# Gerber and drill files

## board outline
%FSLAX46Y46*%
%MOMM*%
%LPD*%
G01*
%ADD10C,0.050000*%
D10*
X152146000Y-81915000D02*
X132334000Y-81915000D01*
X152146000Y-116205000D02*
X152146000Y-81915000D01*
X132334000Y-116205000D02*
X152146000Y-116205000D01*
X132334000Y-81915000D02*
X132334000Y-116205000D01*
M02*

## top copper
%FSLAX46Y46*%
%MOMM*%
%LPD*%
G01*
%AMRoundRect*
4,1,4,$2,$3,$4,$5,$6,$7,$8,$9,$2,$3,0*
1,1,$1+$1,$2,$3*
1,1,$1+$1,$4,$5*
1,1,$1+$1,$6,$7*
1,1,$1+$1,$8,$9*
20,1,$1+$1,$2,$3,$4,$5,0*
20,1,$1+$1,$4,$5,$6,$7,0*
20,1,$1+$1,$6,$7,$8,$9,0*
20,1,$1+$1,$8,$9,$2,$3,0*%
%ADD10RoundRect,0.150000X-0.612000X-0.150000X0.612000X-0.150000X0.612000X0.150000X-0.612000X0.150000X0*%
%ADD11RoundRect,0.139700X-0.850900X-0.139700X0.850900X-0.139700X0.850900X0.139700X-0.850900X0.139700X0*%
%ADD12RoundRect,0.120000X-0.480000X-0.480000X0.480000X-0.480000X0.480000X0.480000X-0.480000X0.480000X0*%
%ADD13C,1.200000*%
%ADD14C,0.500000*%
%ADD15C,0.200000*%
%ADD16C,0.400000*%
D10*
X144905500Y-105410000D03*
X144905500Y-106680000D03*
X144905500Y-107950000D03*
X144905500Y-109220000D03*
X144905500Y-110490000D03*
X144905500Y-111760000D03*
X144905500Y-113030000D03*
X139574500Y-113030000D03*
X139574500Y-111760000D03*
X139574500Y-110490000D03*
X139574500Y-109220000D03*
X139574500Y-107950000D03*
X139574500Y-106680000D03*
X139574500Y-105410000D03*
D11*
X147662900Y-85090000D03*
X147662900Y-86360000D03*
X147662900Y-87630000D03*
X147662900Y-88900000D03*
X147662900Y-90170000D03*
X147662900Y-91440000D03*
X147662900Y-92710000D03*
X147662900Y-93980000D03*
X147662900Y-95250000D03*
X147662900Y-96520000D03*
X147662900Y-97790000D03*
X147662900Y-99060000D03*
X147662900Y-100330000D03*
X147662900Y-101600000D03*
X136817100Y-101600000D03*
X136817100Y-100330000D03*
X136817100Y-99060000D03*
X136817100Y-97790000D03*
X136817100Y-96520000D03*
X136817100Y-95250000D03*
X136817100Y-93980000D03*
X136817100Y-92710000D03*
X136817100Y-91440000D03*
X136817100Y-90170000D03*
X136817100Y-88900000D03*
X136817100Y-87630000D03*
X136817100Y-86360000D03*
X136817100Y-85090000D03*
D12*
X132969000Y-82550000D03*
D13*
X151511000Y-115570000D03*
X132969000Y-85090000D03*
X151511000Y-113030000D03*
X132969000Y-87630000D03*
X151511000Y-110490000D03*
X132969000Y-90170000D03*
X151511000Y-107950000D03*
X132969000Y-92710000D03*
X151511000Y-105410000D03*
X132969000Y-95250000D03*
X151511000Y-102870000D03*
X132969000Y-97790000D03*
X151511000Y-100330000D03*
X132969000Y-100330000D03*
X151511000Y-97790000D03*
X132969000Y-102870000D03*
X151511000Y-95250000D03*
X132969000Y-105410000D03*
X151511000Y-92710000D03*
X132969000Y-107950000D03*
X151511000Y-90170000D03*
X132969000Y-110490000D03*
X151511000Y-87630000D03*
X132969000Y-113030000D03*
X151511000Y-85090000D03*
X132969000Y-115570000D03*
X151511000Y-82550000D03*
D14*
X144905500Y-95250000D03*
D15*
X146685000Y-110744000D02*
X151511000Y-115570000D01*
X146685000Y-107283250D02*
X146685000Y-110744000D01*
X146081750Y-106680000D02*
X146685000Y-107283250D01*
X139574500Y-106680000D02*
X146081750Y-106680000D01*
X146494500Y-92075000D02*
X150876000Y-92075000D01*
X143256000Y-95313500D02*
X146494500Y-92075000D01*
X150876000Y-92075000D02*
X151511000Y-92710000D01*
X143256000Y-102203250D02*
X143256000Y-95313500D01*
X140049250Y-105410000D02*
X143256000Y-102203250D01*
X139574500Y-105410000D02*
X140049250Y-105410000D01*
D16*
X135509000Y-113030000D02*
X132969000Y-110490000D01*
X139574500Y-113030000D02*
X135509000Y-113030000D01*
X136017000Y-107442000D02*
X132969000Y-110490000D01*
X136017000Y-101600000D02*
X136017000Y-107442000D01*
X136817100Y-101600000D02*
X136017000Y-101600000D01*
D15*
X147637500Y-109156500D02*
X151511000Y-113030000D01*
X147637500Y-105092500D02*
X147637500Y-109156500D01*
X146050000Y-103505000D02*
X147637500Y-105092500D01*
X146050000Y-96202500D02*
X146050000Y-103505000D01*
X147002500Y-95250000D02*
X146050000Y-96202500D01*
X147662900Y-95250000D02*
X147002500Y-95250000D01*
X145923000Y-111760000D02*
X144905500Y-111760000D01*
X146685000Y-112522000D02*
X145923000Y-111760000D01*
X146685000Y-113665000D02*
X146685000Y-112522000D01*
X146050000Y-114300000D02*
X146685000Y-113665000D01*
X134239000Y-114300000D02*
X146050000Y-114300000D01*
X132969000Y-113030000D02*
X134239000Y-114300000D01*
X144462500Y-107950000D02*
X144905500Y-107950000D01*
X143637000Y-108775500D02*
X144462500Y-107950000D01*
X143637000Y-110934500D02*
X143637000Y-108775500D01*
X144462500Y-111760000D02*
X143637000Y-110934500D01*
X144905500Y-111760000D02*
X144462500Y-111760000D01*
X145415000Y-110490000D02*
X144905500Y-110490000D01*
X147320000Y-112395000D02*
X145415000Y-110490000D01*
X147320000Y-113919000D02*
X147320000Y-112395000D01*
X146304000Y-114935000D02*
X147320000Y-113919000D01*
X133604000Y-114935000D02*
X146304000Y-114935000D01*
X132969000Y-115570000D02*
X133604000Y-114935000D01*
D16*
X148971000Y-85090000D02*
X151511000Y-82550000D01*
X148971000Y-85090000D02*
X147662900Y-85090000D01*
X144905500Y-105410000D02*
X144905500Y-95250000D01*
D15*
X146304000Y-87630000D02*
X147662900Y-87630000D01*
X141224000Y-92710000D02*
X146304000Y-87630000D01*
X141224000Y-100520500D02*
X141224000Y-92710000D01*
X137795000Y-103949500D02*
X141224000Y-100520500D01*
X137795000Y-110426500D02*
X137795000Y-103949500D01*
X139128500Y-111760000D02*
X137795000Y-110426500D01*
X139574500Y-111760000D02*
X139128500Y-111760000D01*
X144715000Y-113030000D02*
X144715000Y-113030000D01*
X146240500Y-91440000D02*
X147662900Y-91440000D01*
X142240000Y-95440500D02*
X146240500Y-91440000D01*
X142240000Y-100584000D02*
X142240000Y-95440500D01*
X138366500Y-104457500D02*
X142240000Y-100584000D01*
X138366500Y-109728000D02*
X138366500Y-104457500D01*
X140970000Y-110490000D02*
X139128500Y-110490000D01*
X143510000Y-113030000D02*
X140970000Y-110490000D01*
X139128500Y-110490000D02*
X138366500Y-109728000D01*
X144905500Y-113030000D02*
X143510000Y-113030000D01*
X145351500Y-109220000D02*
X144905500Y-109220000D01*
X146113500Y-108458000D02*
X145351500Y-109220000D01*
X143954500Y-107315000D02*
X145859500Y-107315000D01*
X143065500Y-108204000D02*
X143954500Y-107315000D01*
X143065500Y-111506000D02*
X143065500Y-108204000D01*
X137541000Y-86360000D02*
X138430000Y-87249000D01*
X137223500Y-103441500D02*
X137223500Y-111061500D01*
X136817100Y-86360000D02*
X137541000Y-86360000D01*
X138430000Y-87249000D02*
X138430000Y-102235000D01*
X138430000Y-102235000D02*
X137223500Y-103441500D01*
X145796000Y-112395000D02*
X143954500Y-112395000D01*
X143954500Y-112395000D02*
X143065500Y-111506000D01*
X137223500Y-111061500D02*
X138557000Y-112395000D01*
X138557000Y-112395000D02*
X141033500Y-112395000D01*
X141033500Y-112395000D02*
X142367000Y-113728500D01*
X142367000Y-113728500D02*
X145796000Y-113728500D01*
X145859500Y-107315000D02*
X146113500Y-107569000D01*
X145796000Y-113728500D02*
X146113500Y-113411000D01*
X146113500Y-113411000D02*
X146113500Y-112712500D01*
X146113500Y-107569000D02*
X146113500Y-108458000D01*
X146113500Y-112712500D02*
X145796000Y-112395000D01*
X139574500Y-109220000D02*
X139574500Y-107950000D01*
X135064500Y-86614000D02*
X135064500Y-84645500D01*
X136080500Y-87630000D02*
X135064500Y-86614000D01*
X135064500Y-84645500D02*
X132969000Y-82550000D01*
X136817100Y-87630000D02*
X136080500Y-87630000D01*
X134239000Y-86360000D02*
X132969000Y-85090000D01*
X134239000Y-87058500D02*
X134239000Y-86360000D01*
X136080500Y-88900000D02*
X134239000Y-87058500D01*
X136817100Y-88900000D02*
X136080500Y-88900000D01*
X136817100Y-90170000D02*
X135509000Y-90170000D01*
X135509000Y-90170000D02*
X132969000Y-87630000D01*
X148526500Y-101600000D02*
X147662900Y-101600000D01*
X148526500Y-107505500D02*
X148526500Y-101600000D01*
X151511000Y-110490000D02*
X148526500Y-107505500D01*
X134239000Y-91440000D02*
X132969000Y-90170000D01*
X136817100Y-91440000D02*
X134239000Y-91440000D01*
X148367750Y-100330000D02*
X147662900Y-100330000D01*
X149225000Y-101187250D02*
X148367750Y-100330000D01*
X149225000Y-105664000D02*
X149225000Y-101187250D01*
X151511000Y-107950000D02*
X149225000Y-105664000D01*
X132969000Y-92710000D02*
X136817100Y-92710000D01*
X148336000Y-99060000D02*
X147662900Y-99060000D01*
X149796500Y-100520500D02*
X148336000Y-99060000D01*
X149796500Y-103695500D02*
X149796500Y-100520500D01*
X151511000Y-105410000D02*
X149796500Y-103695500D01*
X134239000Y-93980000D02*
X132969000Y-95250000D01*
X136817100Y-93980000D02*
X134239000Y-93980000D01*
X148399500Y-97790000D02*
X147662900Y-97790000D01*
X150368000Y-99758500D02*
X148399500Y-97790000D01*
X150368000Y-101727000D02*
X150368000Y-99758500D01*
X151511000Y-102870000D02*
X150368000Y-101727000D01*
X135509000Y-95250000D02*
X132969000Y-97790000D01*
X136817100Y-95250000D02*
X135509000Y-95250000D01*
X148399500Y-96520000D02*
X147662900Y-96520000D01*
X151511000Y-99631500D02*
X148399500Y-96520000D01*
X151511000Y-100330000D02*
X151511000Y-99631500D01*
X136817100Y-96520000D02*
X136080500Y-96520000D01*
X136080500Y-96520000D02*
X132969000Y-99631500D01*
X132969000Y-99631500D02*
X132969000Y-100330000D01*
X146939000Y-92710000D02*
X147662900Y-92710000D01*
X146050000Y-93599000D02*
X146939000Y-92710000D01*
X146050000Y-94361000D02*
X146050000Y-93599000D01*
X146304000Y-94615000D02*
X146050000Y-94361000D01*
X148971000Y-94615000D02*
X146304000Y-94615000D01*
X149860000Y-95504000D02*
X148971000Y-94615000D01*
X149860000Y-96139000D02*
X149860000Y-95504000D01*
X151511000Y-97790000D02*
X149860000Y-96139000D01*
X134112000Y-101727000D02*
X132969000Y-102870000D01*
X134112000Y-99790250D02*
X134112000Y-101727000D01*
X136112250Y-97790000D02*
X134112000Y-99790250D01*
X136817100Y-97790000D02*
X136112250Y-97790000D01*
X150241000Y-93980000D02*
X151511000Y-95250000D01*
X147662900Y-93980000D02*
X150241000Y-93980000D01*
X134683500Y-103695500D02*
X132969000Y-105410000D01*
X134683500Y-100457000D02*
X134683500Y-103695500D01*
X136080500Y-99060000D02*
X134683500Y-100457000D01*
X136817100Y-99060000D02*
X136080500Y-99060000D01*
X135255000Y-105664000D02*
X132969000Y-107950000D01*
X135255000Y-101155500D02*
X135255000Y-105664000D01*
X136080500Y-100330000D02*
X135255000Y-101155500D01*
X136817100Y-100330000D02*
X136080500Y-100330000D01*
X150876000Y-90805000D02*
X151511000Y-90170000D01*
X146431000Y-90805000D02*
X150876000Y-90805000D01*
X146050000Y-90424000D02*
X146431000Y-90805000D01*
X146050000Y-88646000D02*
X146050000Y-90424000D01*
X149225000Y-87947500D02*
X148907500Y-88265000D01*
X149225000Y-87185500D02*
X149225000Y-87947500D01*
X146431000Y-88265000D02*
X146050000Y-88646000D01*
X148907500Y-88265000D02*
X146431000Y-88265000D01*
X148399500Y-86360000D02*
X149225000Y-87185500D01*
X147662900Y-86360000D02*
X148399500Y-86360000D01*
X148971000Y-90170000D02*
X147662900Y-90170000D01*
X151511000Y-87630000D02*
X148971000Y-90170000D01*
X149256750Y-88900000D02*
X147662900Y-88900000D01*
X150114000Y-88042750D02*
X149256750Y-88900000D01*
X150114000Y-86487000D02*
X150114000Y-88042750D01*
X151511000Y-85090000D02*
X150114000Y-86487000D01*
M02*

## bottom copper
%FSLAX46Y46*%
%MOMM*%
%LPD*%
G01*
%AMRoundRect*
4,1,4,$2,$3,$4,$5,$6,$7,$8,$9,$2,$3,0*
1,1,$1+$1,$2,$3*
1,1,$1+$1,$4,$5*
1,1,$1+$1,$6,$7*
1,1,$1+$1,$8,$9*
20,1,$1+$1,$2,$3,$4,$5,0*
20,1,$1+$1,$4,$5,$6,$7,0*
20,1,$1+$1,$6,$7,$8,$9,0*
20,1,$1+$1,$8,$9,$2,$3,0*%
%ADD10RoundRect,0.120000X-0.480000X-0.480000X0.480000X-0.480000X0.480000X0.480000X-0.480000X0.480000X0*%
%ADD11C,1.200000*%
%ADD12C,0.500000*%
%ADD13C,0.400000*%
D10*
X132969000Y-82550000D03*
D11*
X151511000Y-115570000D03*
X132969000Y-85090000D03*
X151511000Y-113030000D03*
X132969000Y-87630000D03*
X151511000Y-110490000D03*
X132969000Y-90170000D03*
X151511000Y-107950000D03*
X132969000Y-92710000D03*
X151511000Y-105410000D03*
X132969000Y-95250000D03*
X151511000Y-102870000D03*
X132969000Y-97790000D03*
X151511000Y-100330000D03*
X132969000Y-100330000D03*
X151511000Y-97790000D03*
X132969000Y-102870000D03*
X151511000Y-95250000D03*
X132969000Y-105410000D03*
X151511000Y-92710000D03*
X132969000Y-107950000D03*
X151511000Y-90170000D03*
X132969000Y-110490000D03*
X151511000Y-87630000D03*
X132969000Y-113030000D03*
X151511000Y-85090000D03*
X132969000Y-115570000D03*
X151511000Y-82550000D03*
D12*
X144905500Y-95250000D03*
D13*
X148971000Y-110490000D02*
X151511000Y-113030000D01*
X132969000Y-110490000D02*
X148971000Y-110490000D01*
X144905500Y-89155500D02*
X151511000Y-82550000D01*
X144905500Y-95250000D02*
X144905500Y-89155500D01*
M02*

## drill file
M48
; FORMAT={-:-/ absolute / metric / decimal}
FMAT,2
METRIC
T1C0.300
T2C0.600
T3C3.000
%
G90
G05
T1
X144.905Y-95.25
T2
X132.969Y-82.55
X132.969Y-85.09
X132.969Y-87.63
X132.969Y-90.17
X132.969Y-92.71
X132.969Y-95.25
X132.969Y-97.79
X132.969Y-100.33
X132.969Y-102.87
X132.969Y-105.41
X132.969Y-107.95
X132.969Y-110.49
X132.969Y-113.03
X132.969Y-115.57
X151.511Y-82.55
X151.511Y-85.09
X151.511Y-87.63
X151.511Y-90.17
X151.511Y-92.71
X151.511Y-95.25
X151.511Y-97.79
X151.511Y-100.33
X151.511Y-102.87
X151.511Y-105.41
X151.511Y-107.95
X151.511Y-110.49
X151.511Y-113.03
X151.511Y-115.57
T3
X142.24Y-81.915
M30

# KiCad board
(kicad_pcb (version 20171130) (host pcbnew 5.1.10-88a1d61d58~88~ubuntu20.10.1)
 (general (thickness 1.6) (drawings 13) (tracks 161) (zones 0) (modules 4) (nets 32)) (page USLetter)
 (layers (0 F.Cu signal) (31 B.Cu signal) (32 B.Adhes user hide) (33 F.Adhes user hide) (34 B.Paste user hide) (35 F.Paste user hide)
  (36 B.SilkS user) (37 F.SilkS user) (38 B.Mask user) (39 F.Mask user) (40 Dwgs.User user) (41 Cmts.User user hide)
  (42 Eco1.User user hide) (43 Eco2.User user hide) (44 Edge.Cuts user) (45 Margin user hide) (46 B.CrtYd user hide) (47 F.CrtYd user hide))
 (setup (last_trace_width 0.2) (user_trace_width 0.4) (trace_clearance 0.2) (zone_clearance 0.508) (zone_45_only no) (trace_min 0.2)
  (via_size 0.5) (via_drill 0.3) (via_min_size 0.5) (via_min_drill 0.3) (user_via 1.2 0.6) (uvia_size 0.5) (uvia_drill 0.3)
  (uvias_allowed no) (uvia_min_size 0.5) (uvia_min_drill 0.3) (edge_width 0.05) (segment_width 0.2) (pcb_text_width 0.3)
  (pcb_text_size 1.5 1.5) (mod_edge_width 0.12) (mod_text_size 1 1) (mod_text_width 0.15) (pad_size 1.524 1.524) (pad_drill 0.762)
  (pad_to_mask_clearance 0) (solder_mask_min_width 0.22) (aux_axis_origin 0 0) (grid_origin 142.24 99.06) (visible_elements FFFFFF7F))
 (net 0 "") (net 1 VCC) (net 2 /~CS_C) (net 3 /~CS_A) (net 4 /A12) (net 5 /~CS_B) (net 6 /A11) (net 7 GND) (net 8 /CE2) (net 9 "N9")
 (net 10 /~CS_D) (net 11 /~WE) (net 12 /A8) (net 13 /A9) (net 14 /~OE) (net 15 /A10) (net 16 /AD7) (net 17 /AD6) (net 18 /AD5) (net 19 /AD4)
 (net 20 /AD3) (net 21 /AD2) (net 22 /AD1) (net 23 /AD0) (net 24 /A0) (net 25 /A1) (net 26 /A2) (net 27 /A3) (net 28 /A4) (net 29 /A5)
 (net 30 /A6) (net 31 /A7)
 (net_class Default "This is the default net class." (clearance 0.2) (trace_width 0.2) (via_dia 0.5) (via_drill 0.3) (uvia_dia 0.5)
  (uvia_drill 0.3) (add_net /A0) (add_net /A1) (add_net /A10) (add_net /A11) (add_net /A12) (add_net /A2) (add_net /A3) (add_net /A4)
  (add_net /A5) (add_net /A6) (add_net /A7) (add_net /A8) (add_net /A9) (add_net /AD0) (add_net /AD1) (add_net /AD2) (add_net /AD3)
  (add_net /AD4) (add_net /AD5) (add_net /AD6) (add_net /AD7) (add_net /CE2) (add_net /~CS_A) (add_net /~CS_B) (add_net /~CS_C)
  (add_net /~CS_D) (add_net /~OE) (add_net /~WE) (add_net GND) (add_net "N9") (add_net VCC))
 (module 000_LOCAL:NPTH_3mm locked (layer F.Cu) (at 142.24 81.915)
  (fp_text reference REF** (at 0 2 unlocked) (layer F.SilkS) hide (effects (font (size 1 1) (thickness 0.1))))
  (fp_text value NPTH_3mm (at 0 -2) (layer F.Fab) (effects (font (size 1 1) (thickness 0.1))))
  (pad "" np_thru_hole circle (at 0 0) (size 3 3) (drill 3) (layers *.Cu *.Mask)))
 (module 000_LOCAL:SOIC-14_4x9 (layer F.Cu) (at 142.24 109.22)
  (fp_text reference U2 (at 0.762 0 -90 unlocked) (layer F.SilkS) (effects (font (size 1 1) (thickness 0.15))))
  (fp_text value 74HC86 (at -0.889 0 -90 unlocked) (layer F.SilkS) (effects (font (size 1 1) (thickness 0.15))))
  (pad 14 smd roundrect (at 2.6655 -3.81) (size 1.524 0.6) (layers F.Cu F.Paste F.Mask) (roundrect_rratio 0.25) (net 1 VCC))
  (pad 13 smd roundrect (at 2.6655 -2.54) (size 1.524 0.6) (layers F.Cu F.Paste F.Mask) (roundrect_rratio 0.25) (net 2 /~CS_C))
  (pad 12 smd roundrect (at 2.6655 -1.27) (size 1.524 0.6) (layers F.Cu F.Paste F.Mask) (roundrect_rratio 0.25) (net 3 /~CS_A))
  (pad 11 smd roundrect (at 2.6655 0) (size 1.524 0.6) (layers F.Cu F.Paste F.Mask) (roundrect_rratio 0.25) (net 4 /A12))
  (pad 10 smd roundrect (at 2.6655 1.27) (size 1.524 0.6) (layers F.Cu F.Paste F.Mask) (roundrect_rratio 0.25) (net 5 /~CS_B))
  (pad 9 smd roundrect (at 2.6655 2.54) (size 1.524 0.6) (layers F.Cu F.Paste F.Mask) (roundrect_rratio 0.25) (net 3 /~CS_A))
  (pad 8 smd roundrect (at 2.6655 3.81) (size 1.524 0.6) (layers F.Cu F.Paste F.Mask) (roundrect_rratio 0.25) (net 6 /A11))
  (pad 7 smd roundrect (at -2.6655 3.81) (size 1.524 0.6) (layers F.Cu F.Paste F.Mask) (roundrect_rratio 0.25) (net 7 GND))
  (pad 6 smd roundrect (at -2.6655 2.54) (size 1.524 0.6) (layers F.Cu F.Paste F.Mask) (roundrect_rratio 0.25) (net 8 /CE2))
  (pad 5 smd roundrect (at -2.6655 1.27) (size 1.524 0.6) (layers F.Cu F.Paste F.Mask) (roundrect_rratio 0.25) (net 6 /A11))
  (pad 4 smd roundrect (at -2.6655 0) (size 1.524 0.6) (layers F.Cu F.Paste F.Mask) (roundrect_rratio 0.25) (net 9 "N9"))
  (pad 3 smd roundrect (at -2.6655 -1.27) (size 1.524 0.6) (layers F.Cu F.Paste F.Mask) (roundrect_rratio 0.25) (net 9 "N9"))
  (pad 2 smd roundrect (at -2.6655 -2.54) (size 1.524 0.6) (layers F.Cu F.Paste F.Mask) (roundrect_rratio 0.25) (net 2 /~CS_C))
  (pad 1 smd roundrect (at -2.6655 -3.81) (size 1.524 0.6) (layers F.Cu F.Paste F.Mask) (roundrect_rratio 0.25) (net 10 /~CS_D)))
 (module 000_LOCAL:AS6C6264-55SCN (layer F.Cu) (at 142.24 93.345)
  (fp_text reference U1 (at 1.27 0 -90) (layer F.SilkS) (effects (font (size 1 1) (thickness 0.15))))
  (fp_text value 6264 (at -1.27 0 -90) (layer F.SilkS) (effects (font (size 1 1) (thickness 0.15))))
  (pad 28 smd roundrect (at 5.4229 -8.255) (size 1.9812 0.5588) (layers F.Cu F.Paste F.Mask) (roundrect_rratio 0.25) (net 1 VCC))
  (pad 27 smd roundrect (at 5.4229 -6.985) (size 1.9812 0.5588) (layers F.Cu F.Paste F.Mask) (roundrect_rratio 0.25) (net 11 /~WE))
  (pad 26 smd roundrect (at 5.4229 -5.715) (size 1.9812 0.5588) (layers F.Cu F.Paste F.Mask) (roundrect_rratio 0.25) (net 8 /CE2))
  (pad 25 smd roundrect (at 5.4229 -4.445) (size 1.9812 0.5588) (layers F.Cu F.Paste F.Mask) (roundrect_rratio 0.25) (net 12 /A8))
  (pad 24 smd roundrect (at 5.4229 -3.175) (size 1.9812 0.5588) (layers F.Cu F.Paste F.Mask) (roundrect_rratio 0.25) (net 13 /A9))
  (pad 23 smd roundrect (at 5.4229 -1.905) (size 1.9812 0.5588) (layers F.Cu F.Paste F.Mask) (roundrect_rratio 0.25) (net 6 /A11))
  (pad 22 smd roundrect (at 5.4229 -0.635) (size 1.9812 0.5588) (layers F.Cu F.Paste F.Mask) (roundrect_rratio 0.25) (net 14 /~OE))
  (pad 21 smd roundrect (at 5.4229 0.635) (size 1.9812 0.5588) (layers F.Cu F.Paste F.Mask) (roundrect_rratio 0.25) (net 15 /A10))
  (pad 20 smd roundrect (at 5.4229 1.905) (size 1.9812 0.5588) (layers F.Cu F.Paste F.Mask) (roundrect_rratio 0.25) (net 7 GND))
  (pad 19 smd roundrect (at 5.4229 3.175) (size 1.9812 0.5588) (layers F.Cu F.Paste F.Mask) (roundrect_rratio 0.25) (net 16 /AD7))
  (pad 18 smd roundrect (at 5.4229 4.445) (size 1.9812 0.5588) (layers F.Cu F.Paste F.Mask) (roundrect_rratio 0.25) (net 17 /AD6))
  (pad 17 smd roundrect (at 5.4229 5.715) (size 1.9812 0.5588) (layers F.Cu F.Paste F.Mask) (roundrect_rratio 0.25) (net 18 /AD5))
  (pad 16 smd roundrect (at 5.4229 6.985) (size 1.9812 0.5588) (layers F.Cu F.Paste F.Mask) (roundrect_rratio 0.25) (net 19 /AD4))
  (pad 15 smd roundrect (at 5.4229 8.255) (size 1.9812 0.5588) (layers F.Cu F.Paste F.Mask) (roundrect_rratio 0.25) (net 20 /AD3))
  (pad 14 smd roundrect (at -5.4229 8.255) (size 1.9812 0.5588) (layers F.Cu F.Paste F.Mask) (roundrect_rratio 0.25) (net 7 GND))
  (pad 13 smd roundrect (at -5.4229 6.985) (size 1.9812 0.5588) (layers F.Cu F.Paste F.Mask) (roundrect_rratio 0.25) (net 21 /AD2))
  (pad 12 smd roundrect (at -5.4229 5.715) (size 1.9812 0.5588) (layers F.Cu F.Paste F.Mask) (roundrect_rratio 0.25) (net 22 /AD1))
  (pad 11 smd roundrect (at -5.4229 4.445) (size 1.9812 0.5588) (layers F.Cu F.Paste F.Mask) (roundrect_rratio 0.25) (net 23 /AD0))
  (pad 10 smd roundrect (at -5.4229 3.175) (size 1.9812 0.5588) (layers F.Cu F.Paste F.Mask) (roundrect_rratio 0.25) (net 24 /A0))
  (pad 9 smd roundrect (at -5.4229 1.905) (size 1.9812 0.5588) (layers F.Cu F.Paste F.Mask) (roundrect_rratio 0.25) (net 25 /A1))
  (pad 8 smd roundrect (at -5.4229 0.635) (size 1.9812 0.5588) (layers F.Cu F.Paste F.Mask) (roundrect_rratio 0.25) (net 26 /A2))
  (pad 7 smd roundrect (at -5.4229 -0.635) (size 1.9812 0.5588) (layers F.Cu F.Paste F.Mask) (roundrect_rratio 0.25) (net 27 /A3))
  (pad 6 smd roundrect (at -5.4229 -1.905) (size 1.9812 0.5588) (layers F.Cu F.Paste F.Mask) (roundrect_rratio 0.25) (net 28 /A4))
  (pad 5 smd roundrect (at -5.4229 -3.175) (size 1.9812 0.5588) (layers F.Cu F.Paste F.Mask) (roundrect_rratio 0.25) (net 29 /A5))
  (pad 4 smd roundrect (at -5.4229 -4.445) (size 1.9812 0.5588) (layers F.Cu F.Paste F.Mask) (roundrect_rratio 0.25) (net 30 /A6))
  (pad 3 smd roundrect (at -5.4229 -5.715) (size 1.9812 0.5588) (layers F.Cu F.Paste F.Mask) (roundrect_rratio 0.25) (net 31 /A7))
  (pad 2 smd roundrect (at -5.4229 -6.985) (size 1.9812 0.5588) (layers F.Cu F.Paste F.Mask) (roundrect_rratio 0.25) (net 4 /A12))
  (pad 1 smd roundrect (at -5.4229 -8.255) (size 1.9812 0.5588) (layers F.Cu F.Paste F.Mask) (roundrect_rratio 0.25)))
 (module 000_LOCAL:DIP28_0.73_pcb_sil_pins (layer F.Cu) (at 142.24 99.06)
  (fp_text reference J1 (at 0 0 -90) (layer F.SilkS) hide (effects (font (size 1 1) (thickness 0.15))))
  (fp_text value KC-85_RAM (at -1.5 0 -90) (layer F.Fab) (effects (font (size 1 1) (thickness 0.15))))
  (pad 1 thru_hole roundrect (at -9.271 -16.51) (size 1.2 1.2) (drill 0.6) (layers *.Cu *.Mask) (roundrect_rratio 0.1) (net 31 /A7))
  (pad 15 thru_hole circle (at 9.271 16.51) (size 1.2 1.2) (drill 0.6) (layers *.Cu *.Mask) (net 2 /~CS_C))
  (pad 2 thru_hole circle (at -9.271 -13.97) (size 1.2 1.2) (drill 0.6) (layers *.Cu *.Mask) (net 30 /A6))
  (pad 16 thru_hole circle (at 9.271 13.97) (size 1.2 1.2) (drill 0.6) (layers *.Cu *.Mask) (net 7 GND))
  (pad 3 thru_hole circle (at -9.271 -11.43) (size 1.2 1.2) (drill 0.6) (layers *.Cu *.Mask) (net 29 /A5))
  (pad 17 thru_hole circle (at 9.271 11.43) (size 1.2 1.2) (drill 0.6) (layers *.Cu *.Mask) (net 20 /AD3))
  (pad 4 thru_hole circle (at -9.271 -8.89) (size 1.2 1.2) (drill 0.6) (layers *.Cu *.Mask) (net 28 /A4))
  (pad 18 thru_hole circle (at 9.271 8.89) (size 1.2 1.2) (drill 0.6) (layers *.Cu *.Mask) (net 19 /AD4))
  (pad 5 thru_hole circle (at -9.271 -6.35) (size 1.2 1.2) (drill 0.6) (layers *.Cu *.Mask) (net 27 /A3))
  (pad 19 thru_hole circle (at 9.271 6.35) (size 1.2 1.2) (drill 0.6) (layers *.Cu *.Mask) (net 18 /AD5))
  (pad 6 thru_hole circle (at -9.271 -3.81) (size 1.2 1.2) (drill 0.6) (layers *.Cu *.Mask) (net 26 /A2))
  (pad 20 thru_hole circle (at 9.271 3.81) (size 1.2 1.2) (drill 0.6) (layers *.Cu *.Mask) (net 17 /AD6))
  (pad 7 thru_hole circle (at -9.271 -1.27) (size 1.2 1.2) (drill 0.6) (layers *.Cu *.Mask) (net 25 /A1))
  (pad 21 thru_hole circle (at 9.271 1.27) (size 1.2 1.2) (drill 0.6) (layers *.Cu *.Mask) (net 16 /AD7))
  (pad 8 thru_hole circle (at -9.271 1.27) (size 1.2 1.2) (drill 0.6) (layers *.Cu *.Mask) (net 24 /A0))
  (pad 22 thru_hole circle (at 9.271 -1.27) (size 1.2 1.2) (drill 0.6) (layers *.Cu *.Mask) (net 14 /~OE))
  (pad 9 thru_hole circle (at -9.271 3.81) (size 1.2 1.2) (drill 0.6) (layers *.Cu *.Mask) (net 23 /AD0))
  (pad 23 thru_hole circle (at 9.271 -3.81) (size 1.2 1.2) (drill 0.6) (layers *.Cu *.Mask) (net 15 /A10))
  (pad 10 thru_hole circle (at -9.271 6.35) (size 1.2 1.2) (drill 0.6) (layers *.Cu *.Mask) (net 22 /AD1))
  (pad 24 thru_hole circle (at 9.271 -6.35) (size 1.2 1.2) (drill 0.6) (layers *.Cu *.Mask) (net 10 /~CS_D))
  (pad 11 thru_hole circle (at -9.271 8.89) (size 1.2 1.2) (drill 0.6) (layers *.Cu *.Mask) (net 21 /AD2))
  (pad 25 thru_hole circle (at 9.271 -8.89) (size 1.2 1.2) (drill 0.6) (layers *.Cu *.Mask) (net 11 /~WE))
  (pad 12 thru_hole circle (at -9.271 11.43) (size 1.2 1.2) (drill 0.6) (layers *.Cu *.Mask) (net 7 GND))
  (pad 26 thru_hole circle (at 9.271 -11.43) (size 1.2 1.2) (drill 0.6) (layers *.Cu *.Mask) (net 13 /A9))
  (pad 13 thru_hole circle (at -9.271 13.97) (size 1.2 1.2) (drill 0.6) (layers *.Cu *.Mask) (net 3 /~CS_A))
  (pad 27 thru_hole circle (at 9.271 -13.97) (size 1.2 1.2) (drill 0.6) (layers *.Cu *.Mask) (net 12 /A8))
  (pad 14 thru_hole circle (at -9.271 16.51) (size 1.2 1.2) (drill 0.6) (layers *.Cu *.Mask) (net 5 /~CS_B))
  (pad 28 thru_hole circle (at 9.271 -16.51) (size 1.2 1.2) (drill 0.6) (layers *.Cu *.Mask) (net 1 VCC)))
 (gr_line (start 152.146 81.915) (end 132.334 81.915) (layer Edge.Cuts) (width 0.05))
 (gr_line (start 152.146 116.205) (end 152.146 81.915) (layer Edge.Cuts) (width 0.05))
 (gr_line (start 132.334 116.205) (end 152.146 116.205) (layer Edge.Cuts) (width 0.05))
 (gr_line (start 132.334 81.915) (end 132.334 116.205) (layer Edge.Cuts) (width 0.05))
 (segment (start 146.685 110.744) (end 151.511 115.57) (width 0.2) (layer F.Cu) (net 2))
 (segment (start 146.685 107.28325) (end 146.685 110.744) (width 0.2) (layer F.Cu) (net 2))
 (segment (start 146.08175 106.68) (end 146.685 107.28325) (width 0.2) (layer F.Cu) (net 2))
 (segment (start 139.5745 106.68) (end 146.08175 106.68) (width 0.2) (layer F.Cu) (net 2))
 (segment (start 146.4945 92.075) (end 150.876 92.075) (width 0.2) (layer F.Cu) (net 10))
 (segment (start 143.256 95.3135) (end 146.4945 92.075) (width 0.2) (layer F.Cu) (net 10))
 (segment (start 150.876 92.075) (end 151.511 92.71) (width 0.2) (layer F.Cu) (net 10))
 (segment (start 143.256 102.20325) (end 143.256 95.3135) (width 0.2) (layer F.Cu) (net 10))
 (segment (start 140.04925 105.41) (end 143.256 102.20325) (width 0.2) (layer F.Cu) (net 10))
 (segment (start 139.5745 105.41) (end 140.04925 105.41) (width 0.2) (layer F.Cu) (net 10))
 (segment (start 135.509 113.03) (end 132.969 110.49) (width 0.4) (layer F.Cu) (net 7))
 (segment (start 139.5745 113.03) (end 135.509 113.03) (width 0.4) (layer F.Cu) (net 7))
 (segment (start 136.017 107.442) (end 132.969 110.49) (width 0.4) (layer F.Cu) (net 7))
 (segment (start 136.017 101.6) (end 136.017 107.442) (width 0.4) (layer F.Cu) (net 7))
 (segment (start 136.8171 101.6) (end 136.017 101.6) (width 0.4) (layer F.Cu) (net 7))
 (segment (start 147.6375 109.1565) (end 151.511 113.03) (width 0.2) (layer F.Cu) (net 7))
 (segment (start 147.6375 105.0925) (end 147.6375 109.1565) (width 0.2) (layer F.Cu) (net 7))
 (segment (start 146.05 103.505) (end 147.6375 105.0925) (width 0.2) (layer F.Cu) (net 7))
 (segment (start 146.05 96.2025) (end 146.05 103.505) (width 0.2) (layer F.Cu) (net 7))
 (segment (start 147.0025 95.25) (end 146.05 96.2025) (width 0.2) (layer F.Cu) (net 7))
 (segment (start 147.6629 95.25) (end 147.0025 95.25) (width 0.2) (layer F.Cu) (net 7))
 (segment (start 148.971 110.49) (end 151.511 113.03) (width 0.4) (layer B.Cu) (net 7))
 (segment (start 132.969 110.49) (end 148.971 110.49) (width 0.4) (layer B.Cu) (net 7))
 (segment (start 145.923 111.76) (end 144.9055 111.76) (width 0.2) (layer F.Cu) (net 3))
 (segment (start 146.685 112.522) (end 145.923 111.76) (width 0.2) (layer F.Cu) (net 3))
 (segment (start 146.685 113.665) (end 146.685 112.522) (width 0.2) (layer F.Cu) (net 3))
 (segment (start 146.05 114.3) (end 146.685 113.665) (width 0.2) (layer F.Cu) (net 3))
 (segment (start 134.239 114.3) (end 146.05 114.3) (width 0.2) (layer F.Cu) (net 3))
 (segment (start 132.969 113.03) (end 134.239 114.3) (width 0.2) (layer F.Cu) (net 3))
 (segment (start 144.4625 107.95) (end 144.9055 107.95) (width 0.2) (layer F.Cu) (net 3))
 (segment (start 143.637 108.7755) (end 144.4625 107.95) (width 0.2) (layer F.Cu) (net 3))
 (segment (start 143.637 110.9345) (end 143.637 108.7755) (width 0.2) (layer F.Cu) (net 3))
 (segment (start 144.4625 111.76) (end 143.637 110.9345) (width 0.2) (layer F.Cu) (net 3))
 (segment (start 144.9055 111.76) (end 144.4625 111.76) (width 0.2) (layer F.Cu) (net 3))
 (segment (start 145.415 110.49) (end 144.9055 110.49) (width 0.2) (layer F.Cu) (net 5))
 (segment (start 147.32 112.395) (end 145.415 110.49) (width 0.2) (layer F.Cu) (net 5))
 (segment (start 147.32 113.919) (end 147.32 112.395) (width 0.2) (layer F.Cu) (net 5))
 (segment (start 146.304 114.935) (end 147.32 113.919) (width 0.2) (layer F.Cu) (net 5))
 (segment (start 133.604 114.935) (end 146.304 114.935) (width 0.2) (layer F.Cu) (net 5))
 (segment (start 132.969 115.57) (end 133.604 114.935) (width 0.2) (layer F.Cu) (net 5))
 (segment (start 148.971 85.09) (end 151.511 82.55) (width 0.4) (layer F.Cu) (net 1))
 (segment (start 148.971 85.09) (end 147.6629 85.09) (width 0.4) (layer F.Cu) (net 1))
 (segment (start 144.9055 105.41) (end 144.9055 95.25) (width 0.4) (layer F.Cu) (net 1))
 (segment (start 144.9055 89.1555) (end 151.511 82.55) (width 0.4) (layer B.Cu) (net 1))
 (segment (start 144.9055 95.25) (end 144.9055 89.1555) (width 0.4) (layer B.Cu) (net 1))
 (via (at 144.9055 95.25) (size 0.5) (drill 0.3) (layers F.Cu B.Cu) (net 1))
 (segment (start 146.304 87.63) (end 147.6629 87.63) (width 0.2) (layer F.Cu) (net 8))
 (segment (start 141.224 92.71) (end 146.304 87.63) (width 0.2) (layer F.Cu) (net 8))
 (segment (start 141.224 100.5205) (end 141.224 92.71) (width 0.2) (layer F.Cu) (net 8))
 (segment (start 137.795 103.9495) (end 141.224 100.5205) (width 0.2) (layer F.Cu) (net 8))
 (segment (start 137.795 110.4265) (end 137.795 103.9495) (width 0.2) (layer F.Cu) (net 8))
 (segment (start 139.1285 111.76) (end 137.795 110.4265) (width 0.2) (layer F.Cu) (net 8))
 (segment (start 139.5745 111.76) (end 139.1285 111.76) (width 0.2) (layer F.Cu) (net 8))
 (segment (start 144.715 113.03) (end 144.715 113.03) (width 0.2) (layer F.Cu) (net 6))
 (segment (start 146.2405 91.44) (end 147.6629 91.44) (width 0.2) (layer F.Cu) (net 6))
 (segment (start 142.24 95.4405) (end 146.2405 91.44) (width 0.2) (layer F.Cu) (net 6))
 (segment (start 142.24 100.584) (end 142.24 95.4405) (width 0.2) (layer F.Cu) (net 6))
 (segment (start 138.3665 104.4575) (end 142.24 100.584) (width 0.2) (layer F.Cu) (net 6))
 (segment (start 138.3665 109.728) (end 138.3665 104.4575) (width 0.2) (layer F.Cu) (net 6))
 (segment (start 140.97 110.49) (end 139.1285 110.49) (width 0.2) (layer F.Cu) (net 6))
 (segment (start 143.51 113.03) (end 140.97 110.49) (width 0.2) (layer F.Cu) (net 6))
 (segment (start 139.1285 110.49) (end 138.3665 109.728) (width 0.2) (layer F.Cu) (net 6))
 (segment (start 144.9055 113.03) (end 143.51 113.03) (width 0.2) (layer F.Cu) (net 6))
 (segment (start 145.3515 109.22) (end 144.9055 109.22) (width 0.2) (layer F.Cu) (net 4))
 (segment (start 146.1135 108.458) (end 145.3515 109.22) (width 0.2) (layer F.Cu) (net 4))
 (segment (start 143.9545 107.315) (end 145.8595 107.315) (width 0.2) (layer F.Cu) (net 4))
 (segment (start 143.0655 108.204) (end 143.9545 107.315) (width 0.2) (layer F.Cu) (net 4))
 (segment (start 143.0655 111.506) (end 143.0655 108.204) (width 0.2) (layer F.Cu) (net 4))
 (segment (start 137.541 86.36) (end 138.43 87.249) (width 0.2) (layer F.Cu) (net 4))
 (segment (start 137.2235 103.4415) (end 137.2235 111.0615) (width 0.2) (layer F.Cu) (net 4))
 (segment (start 136.8171 86.36) (end 137.541 86.36) (width 0.2) (layer F.Cu) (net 4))
 (segment (start 138.43 87.249) (end 138.43 102.235) (width 0.2) (layer F.Cu) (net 4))
 (segment (start 138.43 102.235) (end 137.2235 103.4415) (width 0.2) (layer F.Cu) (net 4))
 (segment (start 145.796 112.395) (end 143.9545 112.395) (width 0.2) (layer F.Cu) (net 4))
 (segment (start 143.9545 112.395) (end 143.0655 111.506) (width 0.2) (layer F.Cu) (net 4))
 (segment (start 137.2235 111.0615) (end 138.557 112.395) (width 0.2) (layer F.Cu) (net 4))
 (segment (start 138.557 112.395) (end 141.0335 112.395) (width 0.2) (layer F.Cu) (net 4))
 (segment (start 141.0335 112.395) (end 142.367 113.7285) (width 0.2) (layer F.Cu) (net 4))
 (segment (start 142.367 113.7285) (end 145.796 113.7285) (width 0.2) (layer F.Cu) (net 4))
 (segment (start 145.8595 107.315) (end 146.1135 107.569) (width 0.2) (layer F.Cu) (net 4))
 (segment (start 145.796 113.7285) (end 146.1135 113.411) (width 0.2) (layer F.Cu) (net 4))
 (segment (start 146.1135 113.411) (end 146.1135 112.7125) (width 0.2) (layer F.Cu) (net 4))
 (segment (start 146.1135 107.569) (end 146.1135 108.458) (width 0.2) (layer F.Cu) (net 4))
 (segment (start 146.1135 112.7125) (end 145.796 112.395) (width 0.2) (layer F.Cu) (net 4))
 (segment (start 139.5745 109.22) (end 139.5745 107.95) (width 0.2) (layer F.Cu) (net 9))
 (segment (start 135.0645 86.614) (end 135.0645 84.6455) (width 0.2) (layer F.Cu) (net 31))
 (segment (start 136.0805 87.63) (end 135.0645 86.614) (width 0.2) (layer F.Cu) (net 31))
 (segment (start 135.0645 84.6455) (end 132.969 82.55) (width 0.2) (layer F.Cu) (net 31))
 (segment (start 136.8171 87.63) (end 136.0805 87.63) (width 0.2) (layer F.Cu) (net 31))
 (segment (start 134.239 86.36) (end 132.969 85.09) (width 0.2) (layer F.Cu) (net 30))
 (segment (start 134.239 87.0585) (end 134.239 86.36) (width 0.2) (layer F.Cu) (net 30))
 (segment (start 136.0805 88.9) (end 134.239 87.0585) (width 0.2) (layer F.Cu) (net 30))
 (segment (start 136.8171 88.9) (end 136.0805 88.9) (width 0.2) (layer F.Cu) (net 30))
 (segment (start 136.8171 90.17) (end 135.509 90.17) (width 0.2) (layer F.Cu) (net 29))
 (segment (start 135.509 90.17) (end 132.969 87.63) (width 0.2) (layer F.Cu) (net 29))
 (segment (start 148.5265 101.6) (end 147.6629 101.6) (width 0.2) (layer F.Cu) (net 20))
 (segment (start 148.5265 107.5055) (end 148.5265 101.6) (width 0.2) (layer F.Cu) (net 20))
 (segment (start 151.511 110.49) (end 148.5265 107.5055) (width 0.2) (layer F.Cu) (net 20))
 (segment (start 134.239 91.44) (end 132.969 90.17) (width 0.2) (layer F.Cu) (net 28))
 (segment (start 136.8171 91.44) (end 134.239 91.44) (width 0.2) (layer F.Cu) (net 28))
 (segment (start 148.36775 100.33) (end 147.6629 100.33) (width 0.2) (layer F.Cu) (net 19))
 (segment (start 149.225 101.18725) (end 148.36775 100.33) (width 0.2) (layer F.Cu) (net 19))
 (segment (start 149.225 105.664) (end 149.225 101.18725) (width 0.2) (layer F.Cu) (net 19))
 (segment (start 151.511 107.95) (end 149.225 105.664) (width 0.2) (layer F.Cu) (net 19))
 (segment (start 132.969 92.71) (end 136.8171 92.71) (width 0.2) (layer F.Cu) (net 27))
 (segment (start 148.336 99.06) (end 147.6629 99.06) (width 0.2) (layer F.Cu) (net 18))
 (segment (start 149.7965 100.5205) (end 148.336 99.06) (width 0.2) (layer F.Cu) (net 18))
 (segment (start 149.7965 103.6955) (end 149.7965 100.5205) (width 0.2) (layer F.Cu) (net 18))
 (segment (start 151.511 105.41) (end 149.7965 103.6955) (width 0.2) (layer F.Cu) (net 18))
 (segment (start 134.239 93.98) (end 132.969 95.25) (width 0.2) (layer F.Cu) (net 26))
 (segment (start 136.8171 93.98) (end 134.239 93.98) (width 0.2) (layer F.Cu) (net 26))
 (segment (start 148.3995 97.79) (end 147.6629 97.79) (width 0.2) (layer F.Cu) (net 17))
 (segment (start 150.368 99.7585) (end 148.3995 97.79) (width 0.2) (layer F.Cu) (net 17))
 (segment (start 150.368 101.727) (end 150.368 99.7585) (width 0.2) (layer F.Cu) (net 17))
 (segment (start 151.511 102.87) (end 150.368 101.727) (width 0.2) (layer F.Cu) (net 17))
 (segment (start 135.509 95.25) (end 132.969 97.79) (width 0.2) (layer F.Cu) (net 25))
 (segment (start 136.8171 95.25) (end 135.509 95.25) (width 0.2) (layer F.Cu) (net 25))
 (segment (start 148.3995 96.52) (end 147.6629 96.52) (width 0.2) (layer F.Cu) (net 16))
 (segment (start 151.511 99.6315) (end 148.3995 96.52) (width 0.2) (layer F.Cu) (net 16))
 (segment (start 151.511 100.33) (end 151.511 99.6315) (width 0.2) (layer F.Cu) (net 16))
 (segment (start 136.8171 96.52) (end 136.0805 96.52) (width 0.2) (layer F.Cu) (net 24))
 (segment (start 136.0805 96.52) (end 132.969 99.6315) (width 0.2) (layer F.Cu) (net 24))
 (segment (start 132.969 99.6315) (end 132.969 100.33) (width 0.2) (layer F.Cu) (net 24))
 (segment (start 146.939 92.71) (end 147.6629 92.71) (width 0.2) (layer F.Cu) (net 14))
 (segment (start 146.05 93.599) (end 146.939 92.71) (width 0.2) (layer F.Cu) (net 14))
 (segment (start 146.05 94.361) (end 146.05 93.599) (width 0.2) (layer F.Cu) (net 14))
 (segment (start 146.304 94.615) (end 146.05 94.361) (width 0.2) (layer F.Cu) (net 14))
 (segment (start 148.971 94.615) (end 146.304 94.615) (width 0.2) (layer F.Cu) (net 14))
 (segment (start 149.86 95.504) (end 148.971 94.615) (width 0.2) (layer F.Cu) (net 14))
 (segment (start 149.86 96.139) (end 149.86 95.504) (width 0.2) (layer F.Cu) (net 14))
 (segment (start 151.511 97.79) (end 149.86 96.139) (width 0.2) (layer F.Cu) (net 14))
 (segment (start 134.112 101.727) (end 132.969 102.87) (width 0.2) (layer F.Cu) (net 23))
 (segment (start 134.112 99.79025) (end 134.112 101.727) (width 0.2) (layer F.Cu) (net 23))
 (segment (start 136.11225 97.79) (end 134.112 99.79025) (width 0.2) (layer F.Cu) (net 23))
 (segment (start 136.8171 97.79) (end 136.11225 97.79) (width 0.2) (layer F.Cu) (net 23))
 (segment (start 150.241 93.98) (end 151.511 95.25) (width 0.2) (layer F.Cu) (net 15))
 (segment (start 147.6629 93.98) (end 150.241 93.98) (width 0.2) (layer F.Cu) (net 15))
 (segment (start 134.6835 103.6955) (end 132.969 105.41) (width 0.2) (layer F.Cu) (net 22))
 (segment (start 134.6835 100.457) (end 134.6835 103.6955) (width 0.2) (layer F.Cu) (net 22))
 (segment (start 136.0805 99.06) (end 134.6835 100.457) (width 0.2) (layer F.Cu) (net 22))
 (segment (start 136.8171 99.06) (end 136.0805 99.06) (width 0.2) (layer F.Cu) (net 22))
 (segment (start 135.255 105.664) (end 132.969 107.95) (width 0.2) (layer F.Cu) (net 21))
 (segment (start 135.255 101.1555) (end 135.255 105.664) (width 0.2) (layer F.Cu) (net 21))
 (segment (start 136.0805 100.33) (end 135.255 101.1555) (width 0.2) (layer F.Cu) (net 21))
 (segment (start 136.8171 100.33) (end 136.0805 100.33) (width 0.2) (layer F.Cu) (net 21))
 (segment (start 150.876 90.805) (end 151.511 90.17) (width 0.2) (layer F.Cu) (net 11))
 (segment (start 146.431 90.805) (end 150.876 90.805) (width 0.2) (layer F.Cu) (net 11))
 (segment (start 146.05 90.424) (end 146.431 90.805) (width 0.2) (layer F.Cu) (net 11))
 (segment (start 146.05 88.646) (end 146.05 90.424) (width 0.2) (layer F.Cu) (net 11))
 (segment (start 149.225 87.9475) (end 148.9075 88.265) (width 0.2) (layer F.Cu) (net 11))
 (segment (start 149.225 87.1855) (end 149.225 87.9475) (width 0.2) (layer F.Cu) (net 11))
 (segment (start 146.431 88.265) (end 146.05 88.646) (width 0.2) (layer F.Cu) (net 11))
 (segment (start 148.9075 88.265) (end 146.431 88.265) (width 0.2) (layer F.Cu) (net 11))
 (segment (start 148.3995 86.36) (end 149.225 87.1855) (width 0.2) (layer F.Cu) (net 11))
 (segment (start 147.6629 86.36) (end 148.3995 86.36) (width 0.2) (layer F.Cu) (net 11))
 (segment (start 148.971 90.17) (end 147.6629 90.17) (width 0.2) (layer F.Cu) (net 13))
 (segment (start 151.511 87.63) (end 148.971 90.17) (width 0.2) (layer F.Cu) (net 13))
 (segment (start 149.25675 88.9) (end 147.6629 88.9) (width 0.2) (layer F.Cu) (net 12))
 (segment (start 150.114 88.04275) (end 149.25675 88.9) (width 0.2) (layer F.Cu) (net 12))
 (segment (start 150.114 86.487) (end 150.114 88.04275) (width 0.2) (layer F.Cu) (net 12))
 (segment (start 151.511 85.09) (end 150.114 86.487) (width 0.2) (layer F.Cu) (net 12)))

